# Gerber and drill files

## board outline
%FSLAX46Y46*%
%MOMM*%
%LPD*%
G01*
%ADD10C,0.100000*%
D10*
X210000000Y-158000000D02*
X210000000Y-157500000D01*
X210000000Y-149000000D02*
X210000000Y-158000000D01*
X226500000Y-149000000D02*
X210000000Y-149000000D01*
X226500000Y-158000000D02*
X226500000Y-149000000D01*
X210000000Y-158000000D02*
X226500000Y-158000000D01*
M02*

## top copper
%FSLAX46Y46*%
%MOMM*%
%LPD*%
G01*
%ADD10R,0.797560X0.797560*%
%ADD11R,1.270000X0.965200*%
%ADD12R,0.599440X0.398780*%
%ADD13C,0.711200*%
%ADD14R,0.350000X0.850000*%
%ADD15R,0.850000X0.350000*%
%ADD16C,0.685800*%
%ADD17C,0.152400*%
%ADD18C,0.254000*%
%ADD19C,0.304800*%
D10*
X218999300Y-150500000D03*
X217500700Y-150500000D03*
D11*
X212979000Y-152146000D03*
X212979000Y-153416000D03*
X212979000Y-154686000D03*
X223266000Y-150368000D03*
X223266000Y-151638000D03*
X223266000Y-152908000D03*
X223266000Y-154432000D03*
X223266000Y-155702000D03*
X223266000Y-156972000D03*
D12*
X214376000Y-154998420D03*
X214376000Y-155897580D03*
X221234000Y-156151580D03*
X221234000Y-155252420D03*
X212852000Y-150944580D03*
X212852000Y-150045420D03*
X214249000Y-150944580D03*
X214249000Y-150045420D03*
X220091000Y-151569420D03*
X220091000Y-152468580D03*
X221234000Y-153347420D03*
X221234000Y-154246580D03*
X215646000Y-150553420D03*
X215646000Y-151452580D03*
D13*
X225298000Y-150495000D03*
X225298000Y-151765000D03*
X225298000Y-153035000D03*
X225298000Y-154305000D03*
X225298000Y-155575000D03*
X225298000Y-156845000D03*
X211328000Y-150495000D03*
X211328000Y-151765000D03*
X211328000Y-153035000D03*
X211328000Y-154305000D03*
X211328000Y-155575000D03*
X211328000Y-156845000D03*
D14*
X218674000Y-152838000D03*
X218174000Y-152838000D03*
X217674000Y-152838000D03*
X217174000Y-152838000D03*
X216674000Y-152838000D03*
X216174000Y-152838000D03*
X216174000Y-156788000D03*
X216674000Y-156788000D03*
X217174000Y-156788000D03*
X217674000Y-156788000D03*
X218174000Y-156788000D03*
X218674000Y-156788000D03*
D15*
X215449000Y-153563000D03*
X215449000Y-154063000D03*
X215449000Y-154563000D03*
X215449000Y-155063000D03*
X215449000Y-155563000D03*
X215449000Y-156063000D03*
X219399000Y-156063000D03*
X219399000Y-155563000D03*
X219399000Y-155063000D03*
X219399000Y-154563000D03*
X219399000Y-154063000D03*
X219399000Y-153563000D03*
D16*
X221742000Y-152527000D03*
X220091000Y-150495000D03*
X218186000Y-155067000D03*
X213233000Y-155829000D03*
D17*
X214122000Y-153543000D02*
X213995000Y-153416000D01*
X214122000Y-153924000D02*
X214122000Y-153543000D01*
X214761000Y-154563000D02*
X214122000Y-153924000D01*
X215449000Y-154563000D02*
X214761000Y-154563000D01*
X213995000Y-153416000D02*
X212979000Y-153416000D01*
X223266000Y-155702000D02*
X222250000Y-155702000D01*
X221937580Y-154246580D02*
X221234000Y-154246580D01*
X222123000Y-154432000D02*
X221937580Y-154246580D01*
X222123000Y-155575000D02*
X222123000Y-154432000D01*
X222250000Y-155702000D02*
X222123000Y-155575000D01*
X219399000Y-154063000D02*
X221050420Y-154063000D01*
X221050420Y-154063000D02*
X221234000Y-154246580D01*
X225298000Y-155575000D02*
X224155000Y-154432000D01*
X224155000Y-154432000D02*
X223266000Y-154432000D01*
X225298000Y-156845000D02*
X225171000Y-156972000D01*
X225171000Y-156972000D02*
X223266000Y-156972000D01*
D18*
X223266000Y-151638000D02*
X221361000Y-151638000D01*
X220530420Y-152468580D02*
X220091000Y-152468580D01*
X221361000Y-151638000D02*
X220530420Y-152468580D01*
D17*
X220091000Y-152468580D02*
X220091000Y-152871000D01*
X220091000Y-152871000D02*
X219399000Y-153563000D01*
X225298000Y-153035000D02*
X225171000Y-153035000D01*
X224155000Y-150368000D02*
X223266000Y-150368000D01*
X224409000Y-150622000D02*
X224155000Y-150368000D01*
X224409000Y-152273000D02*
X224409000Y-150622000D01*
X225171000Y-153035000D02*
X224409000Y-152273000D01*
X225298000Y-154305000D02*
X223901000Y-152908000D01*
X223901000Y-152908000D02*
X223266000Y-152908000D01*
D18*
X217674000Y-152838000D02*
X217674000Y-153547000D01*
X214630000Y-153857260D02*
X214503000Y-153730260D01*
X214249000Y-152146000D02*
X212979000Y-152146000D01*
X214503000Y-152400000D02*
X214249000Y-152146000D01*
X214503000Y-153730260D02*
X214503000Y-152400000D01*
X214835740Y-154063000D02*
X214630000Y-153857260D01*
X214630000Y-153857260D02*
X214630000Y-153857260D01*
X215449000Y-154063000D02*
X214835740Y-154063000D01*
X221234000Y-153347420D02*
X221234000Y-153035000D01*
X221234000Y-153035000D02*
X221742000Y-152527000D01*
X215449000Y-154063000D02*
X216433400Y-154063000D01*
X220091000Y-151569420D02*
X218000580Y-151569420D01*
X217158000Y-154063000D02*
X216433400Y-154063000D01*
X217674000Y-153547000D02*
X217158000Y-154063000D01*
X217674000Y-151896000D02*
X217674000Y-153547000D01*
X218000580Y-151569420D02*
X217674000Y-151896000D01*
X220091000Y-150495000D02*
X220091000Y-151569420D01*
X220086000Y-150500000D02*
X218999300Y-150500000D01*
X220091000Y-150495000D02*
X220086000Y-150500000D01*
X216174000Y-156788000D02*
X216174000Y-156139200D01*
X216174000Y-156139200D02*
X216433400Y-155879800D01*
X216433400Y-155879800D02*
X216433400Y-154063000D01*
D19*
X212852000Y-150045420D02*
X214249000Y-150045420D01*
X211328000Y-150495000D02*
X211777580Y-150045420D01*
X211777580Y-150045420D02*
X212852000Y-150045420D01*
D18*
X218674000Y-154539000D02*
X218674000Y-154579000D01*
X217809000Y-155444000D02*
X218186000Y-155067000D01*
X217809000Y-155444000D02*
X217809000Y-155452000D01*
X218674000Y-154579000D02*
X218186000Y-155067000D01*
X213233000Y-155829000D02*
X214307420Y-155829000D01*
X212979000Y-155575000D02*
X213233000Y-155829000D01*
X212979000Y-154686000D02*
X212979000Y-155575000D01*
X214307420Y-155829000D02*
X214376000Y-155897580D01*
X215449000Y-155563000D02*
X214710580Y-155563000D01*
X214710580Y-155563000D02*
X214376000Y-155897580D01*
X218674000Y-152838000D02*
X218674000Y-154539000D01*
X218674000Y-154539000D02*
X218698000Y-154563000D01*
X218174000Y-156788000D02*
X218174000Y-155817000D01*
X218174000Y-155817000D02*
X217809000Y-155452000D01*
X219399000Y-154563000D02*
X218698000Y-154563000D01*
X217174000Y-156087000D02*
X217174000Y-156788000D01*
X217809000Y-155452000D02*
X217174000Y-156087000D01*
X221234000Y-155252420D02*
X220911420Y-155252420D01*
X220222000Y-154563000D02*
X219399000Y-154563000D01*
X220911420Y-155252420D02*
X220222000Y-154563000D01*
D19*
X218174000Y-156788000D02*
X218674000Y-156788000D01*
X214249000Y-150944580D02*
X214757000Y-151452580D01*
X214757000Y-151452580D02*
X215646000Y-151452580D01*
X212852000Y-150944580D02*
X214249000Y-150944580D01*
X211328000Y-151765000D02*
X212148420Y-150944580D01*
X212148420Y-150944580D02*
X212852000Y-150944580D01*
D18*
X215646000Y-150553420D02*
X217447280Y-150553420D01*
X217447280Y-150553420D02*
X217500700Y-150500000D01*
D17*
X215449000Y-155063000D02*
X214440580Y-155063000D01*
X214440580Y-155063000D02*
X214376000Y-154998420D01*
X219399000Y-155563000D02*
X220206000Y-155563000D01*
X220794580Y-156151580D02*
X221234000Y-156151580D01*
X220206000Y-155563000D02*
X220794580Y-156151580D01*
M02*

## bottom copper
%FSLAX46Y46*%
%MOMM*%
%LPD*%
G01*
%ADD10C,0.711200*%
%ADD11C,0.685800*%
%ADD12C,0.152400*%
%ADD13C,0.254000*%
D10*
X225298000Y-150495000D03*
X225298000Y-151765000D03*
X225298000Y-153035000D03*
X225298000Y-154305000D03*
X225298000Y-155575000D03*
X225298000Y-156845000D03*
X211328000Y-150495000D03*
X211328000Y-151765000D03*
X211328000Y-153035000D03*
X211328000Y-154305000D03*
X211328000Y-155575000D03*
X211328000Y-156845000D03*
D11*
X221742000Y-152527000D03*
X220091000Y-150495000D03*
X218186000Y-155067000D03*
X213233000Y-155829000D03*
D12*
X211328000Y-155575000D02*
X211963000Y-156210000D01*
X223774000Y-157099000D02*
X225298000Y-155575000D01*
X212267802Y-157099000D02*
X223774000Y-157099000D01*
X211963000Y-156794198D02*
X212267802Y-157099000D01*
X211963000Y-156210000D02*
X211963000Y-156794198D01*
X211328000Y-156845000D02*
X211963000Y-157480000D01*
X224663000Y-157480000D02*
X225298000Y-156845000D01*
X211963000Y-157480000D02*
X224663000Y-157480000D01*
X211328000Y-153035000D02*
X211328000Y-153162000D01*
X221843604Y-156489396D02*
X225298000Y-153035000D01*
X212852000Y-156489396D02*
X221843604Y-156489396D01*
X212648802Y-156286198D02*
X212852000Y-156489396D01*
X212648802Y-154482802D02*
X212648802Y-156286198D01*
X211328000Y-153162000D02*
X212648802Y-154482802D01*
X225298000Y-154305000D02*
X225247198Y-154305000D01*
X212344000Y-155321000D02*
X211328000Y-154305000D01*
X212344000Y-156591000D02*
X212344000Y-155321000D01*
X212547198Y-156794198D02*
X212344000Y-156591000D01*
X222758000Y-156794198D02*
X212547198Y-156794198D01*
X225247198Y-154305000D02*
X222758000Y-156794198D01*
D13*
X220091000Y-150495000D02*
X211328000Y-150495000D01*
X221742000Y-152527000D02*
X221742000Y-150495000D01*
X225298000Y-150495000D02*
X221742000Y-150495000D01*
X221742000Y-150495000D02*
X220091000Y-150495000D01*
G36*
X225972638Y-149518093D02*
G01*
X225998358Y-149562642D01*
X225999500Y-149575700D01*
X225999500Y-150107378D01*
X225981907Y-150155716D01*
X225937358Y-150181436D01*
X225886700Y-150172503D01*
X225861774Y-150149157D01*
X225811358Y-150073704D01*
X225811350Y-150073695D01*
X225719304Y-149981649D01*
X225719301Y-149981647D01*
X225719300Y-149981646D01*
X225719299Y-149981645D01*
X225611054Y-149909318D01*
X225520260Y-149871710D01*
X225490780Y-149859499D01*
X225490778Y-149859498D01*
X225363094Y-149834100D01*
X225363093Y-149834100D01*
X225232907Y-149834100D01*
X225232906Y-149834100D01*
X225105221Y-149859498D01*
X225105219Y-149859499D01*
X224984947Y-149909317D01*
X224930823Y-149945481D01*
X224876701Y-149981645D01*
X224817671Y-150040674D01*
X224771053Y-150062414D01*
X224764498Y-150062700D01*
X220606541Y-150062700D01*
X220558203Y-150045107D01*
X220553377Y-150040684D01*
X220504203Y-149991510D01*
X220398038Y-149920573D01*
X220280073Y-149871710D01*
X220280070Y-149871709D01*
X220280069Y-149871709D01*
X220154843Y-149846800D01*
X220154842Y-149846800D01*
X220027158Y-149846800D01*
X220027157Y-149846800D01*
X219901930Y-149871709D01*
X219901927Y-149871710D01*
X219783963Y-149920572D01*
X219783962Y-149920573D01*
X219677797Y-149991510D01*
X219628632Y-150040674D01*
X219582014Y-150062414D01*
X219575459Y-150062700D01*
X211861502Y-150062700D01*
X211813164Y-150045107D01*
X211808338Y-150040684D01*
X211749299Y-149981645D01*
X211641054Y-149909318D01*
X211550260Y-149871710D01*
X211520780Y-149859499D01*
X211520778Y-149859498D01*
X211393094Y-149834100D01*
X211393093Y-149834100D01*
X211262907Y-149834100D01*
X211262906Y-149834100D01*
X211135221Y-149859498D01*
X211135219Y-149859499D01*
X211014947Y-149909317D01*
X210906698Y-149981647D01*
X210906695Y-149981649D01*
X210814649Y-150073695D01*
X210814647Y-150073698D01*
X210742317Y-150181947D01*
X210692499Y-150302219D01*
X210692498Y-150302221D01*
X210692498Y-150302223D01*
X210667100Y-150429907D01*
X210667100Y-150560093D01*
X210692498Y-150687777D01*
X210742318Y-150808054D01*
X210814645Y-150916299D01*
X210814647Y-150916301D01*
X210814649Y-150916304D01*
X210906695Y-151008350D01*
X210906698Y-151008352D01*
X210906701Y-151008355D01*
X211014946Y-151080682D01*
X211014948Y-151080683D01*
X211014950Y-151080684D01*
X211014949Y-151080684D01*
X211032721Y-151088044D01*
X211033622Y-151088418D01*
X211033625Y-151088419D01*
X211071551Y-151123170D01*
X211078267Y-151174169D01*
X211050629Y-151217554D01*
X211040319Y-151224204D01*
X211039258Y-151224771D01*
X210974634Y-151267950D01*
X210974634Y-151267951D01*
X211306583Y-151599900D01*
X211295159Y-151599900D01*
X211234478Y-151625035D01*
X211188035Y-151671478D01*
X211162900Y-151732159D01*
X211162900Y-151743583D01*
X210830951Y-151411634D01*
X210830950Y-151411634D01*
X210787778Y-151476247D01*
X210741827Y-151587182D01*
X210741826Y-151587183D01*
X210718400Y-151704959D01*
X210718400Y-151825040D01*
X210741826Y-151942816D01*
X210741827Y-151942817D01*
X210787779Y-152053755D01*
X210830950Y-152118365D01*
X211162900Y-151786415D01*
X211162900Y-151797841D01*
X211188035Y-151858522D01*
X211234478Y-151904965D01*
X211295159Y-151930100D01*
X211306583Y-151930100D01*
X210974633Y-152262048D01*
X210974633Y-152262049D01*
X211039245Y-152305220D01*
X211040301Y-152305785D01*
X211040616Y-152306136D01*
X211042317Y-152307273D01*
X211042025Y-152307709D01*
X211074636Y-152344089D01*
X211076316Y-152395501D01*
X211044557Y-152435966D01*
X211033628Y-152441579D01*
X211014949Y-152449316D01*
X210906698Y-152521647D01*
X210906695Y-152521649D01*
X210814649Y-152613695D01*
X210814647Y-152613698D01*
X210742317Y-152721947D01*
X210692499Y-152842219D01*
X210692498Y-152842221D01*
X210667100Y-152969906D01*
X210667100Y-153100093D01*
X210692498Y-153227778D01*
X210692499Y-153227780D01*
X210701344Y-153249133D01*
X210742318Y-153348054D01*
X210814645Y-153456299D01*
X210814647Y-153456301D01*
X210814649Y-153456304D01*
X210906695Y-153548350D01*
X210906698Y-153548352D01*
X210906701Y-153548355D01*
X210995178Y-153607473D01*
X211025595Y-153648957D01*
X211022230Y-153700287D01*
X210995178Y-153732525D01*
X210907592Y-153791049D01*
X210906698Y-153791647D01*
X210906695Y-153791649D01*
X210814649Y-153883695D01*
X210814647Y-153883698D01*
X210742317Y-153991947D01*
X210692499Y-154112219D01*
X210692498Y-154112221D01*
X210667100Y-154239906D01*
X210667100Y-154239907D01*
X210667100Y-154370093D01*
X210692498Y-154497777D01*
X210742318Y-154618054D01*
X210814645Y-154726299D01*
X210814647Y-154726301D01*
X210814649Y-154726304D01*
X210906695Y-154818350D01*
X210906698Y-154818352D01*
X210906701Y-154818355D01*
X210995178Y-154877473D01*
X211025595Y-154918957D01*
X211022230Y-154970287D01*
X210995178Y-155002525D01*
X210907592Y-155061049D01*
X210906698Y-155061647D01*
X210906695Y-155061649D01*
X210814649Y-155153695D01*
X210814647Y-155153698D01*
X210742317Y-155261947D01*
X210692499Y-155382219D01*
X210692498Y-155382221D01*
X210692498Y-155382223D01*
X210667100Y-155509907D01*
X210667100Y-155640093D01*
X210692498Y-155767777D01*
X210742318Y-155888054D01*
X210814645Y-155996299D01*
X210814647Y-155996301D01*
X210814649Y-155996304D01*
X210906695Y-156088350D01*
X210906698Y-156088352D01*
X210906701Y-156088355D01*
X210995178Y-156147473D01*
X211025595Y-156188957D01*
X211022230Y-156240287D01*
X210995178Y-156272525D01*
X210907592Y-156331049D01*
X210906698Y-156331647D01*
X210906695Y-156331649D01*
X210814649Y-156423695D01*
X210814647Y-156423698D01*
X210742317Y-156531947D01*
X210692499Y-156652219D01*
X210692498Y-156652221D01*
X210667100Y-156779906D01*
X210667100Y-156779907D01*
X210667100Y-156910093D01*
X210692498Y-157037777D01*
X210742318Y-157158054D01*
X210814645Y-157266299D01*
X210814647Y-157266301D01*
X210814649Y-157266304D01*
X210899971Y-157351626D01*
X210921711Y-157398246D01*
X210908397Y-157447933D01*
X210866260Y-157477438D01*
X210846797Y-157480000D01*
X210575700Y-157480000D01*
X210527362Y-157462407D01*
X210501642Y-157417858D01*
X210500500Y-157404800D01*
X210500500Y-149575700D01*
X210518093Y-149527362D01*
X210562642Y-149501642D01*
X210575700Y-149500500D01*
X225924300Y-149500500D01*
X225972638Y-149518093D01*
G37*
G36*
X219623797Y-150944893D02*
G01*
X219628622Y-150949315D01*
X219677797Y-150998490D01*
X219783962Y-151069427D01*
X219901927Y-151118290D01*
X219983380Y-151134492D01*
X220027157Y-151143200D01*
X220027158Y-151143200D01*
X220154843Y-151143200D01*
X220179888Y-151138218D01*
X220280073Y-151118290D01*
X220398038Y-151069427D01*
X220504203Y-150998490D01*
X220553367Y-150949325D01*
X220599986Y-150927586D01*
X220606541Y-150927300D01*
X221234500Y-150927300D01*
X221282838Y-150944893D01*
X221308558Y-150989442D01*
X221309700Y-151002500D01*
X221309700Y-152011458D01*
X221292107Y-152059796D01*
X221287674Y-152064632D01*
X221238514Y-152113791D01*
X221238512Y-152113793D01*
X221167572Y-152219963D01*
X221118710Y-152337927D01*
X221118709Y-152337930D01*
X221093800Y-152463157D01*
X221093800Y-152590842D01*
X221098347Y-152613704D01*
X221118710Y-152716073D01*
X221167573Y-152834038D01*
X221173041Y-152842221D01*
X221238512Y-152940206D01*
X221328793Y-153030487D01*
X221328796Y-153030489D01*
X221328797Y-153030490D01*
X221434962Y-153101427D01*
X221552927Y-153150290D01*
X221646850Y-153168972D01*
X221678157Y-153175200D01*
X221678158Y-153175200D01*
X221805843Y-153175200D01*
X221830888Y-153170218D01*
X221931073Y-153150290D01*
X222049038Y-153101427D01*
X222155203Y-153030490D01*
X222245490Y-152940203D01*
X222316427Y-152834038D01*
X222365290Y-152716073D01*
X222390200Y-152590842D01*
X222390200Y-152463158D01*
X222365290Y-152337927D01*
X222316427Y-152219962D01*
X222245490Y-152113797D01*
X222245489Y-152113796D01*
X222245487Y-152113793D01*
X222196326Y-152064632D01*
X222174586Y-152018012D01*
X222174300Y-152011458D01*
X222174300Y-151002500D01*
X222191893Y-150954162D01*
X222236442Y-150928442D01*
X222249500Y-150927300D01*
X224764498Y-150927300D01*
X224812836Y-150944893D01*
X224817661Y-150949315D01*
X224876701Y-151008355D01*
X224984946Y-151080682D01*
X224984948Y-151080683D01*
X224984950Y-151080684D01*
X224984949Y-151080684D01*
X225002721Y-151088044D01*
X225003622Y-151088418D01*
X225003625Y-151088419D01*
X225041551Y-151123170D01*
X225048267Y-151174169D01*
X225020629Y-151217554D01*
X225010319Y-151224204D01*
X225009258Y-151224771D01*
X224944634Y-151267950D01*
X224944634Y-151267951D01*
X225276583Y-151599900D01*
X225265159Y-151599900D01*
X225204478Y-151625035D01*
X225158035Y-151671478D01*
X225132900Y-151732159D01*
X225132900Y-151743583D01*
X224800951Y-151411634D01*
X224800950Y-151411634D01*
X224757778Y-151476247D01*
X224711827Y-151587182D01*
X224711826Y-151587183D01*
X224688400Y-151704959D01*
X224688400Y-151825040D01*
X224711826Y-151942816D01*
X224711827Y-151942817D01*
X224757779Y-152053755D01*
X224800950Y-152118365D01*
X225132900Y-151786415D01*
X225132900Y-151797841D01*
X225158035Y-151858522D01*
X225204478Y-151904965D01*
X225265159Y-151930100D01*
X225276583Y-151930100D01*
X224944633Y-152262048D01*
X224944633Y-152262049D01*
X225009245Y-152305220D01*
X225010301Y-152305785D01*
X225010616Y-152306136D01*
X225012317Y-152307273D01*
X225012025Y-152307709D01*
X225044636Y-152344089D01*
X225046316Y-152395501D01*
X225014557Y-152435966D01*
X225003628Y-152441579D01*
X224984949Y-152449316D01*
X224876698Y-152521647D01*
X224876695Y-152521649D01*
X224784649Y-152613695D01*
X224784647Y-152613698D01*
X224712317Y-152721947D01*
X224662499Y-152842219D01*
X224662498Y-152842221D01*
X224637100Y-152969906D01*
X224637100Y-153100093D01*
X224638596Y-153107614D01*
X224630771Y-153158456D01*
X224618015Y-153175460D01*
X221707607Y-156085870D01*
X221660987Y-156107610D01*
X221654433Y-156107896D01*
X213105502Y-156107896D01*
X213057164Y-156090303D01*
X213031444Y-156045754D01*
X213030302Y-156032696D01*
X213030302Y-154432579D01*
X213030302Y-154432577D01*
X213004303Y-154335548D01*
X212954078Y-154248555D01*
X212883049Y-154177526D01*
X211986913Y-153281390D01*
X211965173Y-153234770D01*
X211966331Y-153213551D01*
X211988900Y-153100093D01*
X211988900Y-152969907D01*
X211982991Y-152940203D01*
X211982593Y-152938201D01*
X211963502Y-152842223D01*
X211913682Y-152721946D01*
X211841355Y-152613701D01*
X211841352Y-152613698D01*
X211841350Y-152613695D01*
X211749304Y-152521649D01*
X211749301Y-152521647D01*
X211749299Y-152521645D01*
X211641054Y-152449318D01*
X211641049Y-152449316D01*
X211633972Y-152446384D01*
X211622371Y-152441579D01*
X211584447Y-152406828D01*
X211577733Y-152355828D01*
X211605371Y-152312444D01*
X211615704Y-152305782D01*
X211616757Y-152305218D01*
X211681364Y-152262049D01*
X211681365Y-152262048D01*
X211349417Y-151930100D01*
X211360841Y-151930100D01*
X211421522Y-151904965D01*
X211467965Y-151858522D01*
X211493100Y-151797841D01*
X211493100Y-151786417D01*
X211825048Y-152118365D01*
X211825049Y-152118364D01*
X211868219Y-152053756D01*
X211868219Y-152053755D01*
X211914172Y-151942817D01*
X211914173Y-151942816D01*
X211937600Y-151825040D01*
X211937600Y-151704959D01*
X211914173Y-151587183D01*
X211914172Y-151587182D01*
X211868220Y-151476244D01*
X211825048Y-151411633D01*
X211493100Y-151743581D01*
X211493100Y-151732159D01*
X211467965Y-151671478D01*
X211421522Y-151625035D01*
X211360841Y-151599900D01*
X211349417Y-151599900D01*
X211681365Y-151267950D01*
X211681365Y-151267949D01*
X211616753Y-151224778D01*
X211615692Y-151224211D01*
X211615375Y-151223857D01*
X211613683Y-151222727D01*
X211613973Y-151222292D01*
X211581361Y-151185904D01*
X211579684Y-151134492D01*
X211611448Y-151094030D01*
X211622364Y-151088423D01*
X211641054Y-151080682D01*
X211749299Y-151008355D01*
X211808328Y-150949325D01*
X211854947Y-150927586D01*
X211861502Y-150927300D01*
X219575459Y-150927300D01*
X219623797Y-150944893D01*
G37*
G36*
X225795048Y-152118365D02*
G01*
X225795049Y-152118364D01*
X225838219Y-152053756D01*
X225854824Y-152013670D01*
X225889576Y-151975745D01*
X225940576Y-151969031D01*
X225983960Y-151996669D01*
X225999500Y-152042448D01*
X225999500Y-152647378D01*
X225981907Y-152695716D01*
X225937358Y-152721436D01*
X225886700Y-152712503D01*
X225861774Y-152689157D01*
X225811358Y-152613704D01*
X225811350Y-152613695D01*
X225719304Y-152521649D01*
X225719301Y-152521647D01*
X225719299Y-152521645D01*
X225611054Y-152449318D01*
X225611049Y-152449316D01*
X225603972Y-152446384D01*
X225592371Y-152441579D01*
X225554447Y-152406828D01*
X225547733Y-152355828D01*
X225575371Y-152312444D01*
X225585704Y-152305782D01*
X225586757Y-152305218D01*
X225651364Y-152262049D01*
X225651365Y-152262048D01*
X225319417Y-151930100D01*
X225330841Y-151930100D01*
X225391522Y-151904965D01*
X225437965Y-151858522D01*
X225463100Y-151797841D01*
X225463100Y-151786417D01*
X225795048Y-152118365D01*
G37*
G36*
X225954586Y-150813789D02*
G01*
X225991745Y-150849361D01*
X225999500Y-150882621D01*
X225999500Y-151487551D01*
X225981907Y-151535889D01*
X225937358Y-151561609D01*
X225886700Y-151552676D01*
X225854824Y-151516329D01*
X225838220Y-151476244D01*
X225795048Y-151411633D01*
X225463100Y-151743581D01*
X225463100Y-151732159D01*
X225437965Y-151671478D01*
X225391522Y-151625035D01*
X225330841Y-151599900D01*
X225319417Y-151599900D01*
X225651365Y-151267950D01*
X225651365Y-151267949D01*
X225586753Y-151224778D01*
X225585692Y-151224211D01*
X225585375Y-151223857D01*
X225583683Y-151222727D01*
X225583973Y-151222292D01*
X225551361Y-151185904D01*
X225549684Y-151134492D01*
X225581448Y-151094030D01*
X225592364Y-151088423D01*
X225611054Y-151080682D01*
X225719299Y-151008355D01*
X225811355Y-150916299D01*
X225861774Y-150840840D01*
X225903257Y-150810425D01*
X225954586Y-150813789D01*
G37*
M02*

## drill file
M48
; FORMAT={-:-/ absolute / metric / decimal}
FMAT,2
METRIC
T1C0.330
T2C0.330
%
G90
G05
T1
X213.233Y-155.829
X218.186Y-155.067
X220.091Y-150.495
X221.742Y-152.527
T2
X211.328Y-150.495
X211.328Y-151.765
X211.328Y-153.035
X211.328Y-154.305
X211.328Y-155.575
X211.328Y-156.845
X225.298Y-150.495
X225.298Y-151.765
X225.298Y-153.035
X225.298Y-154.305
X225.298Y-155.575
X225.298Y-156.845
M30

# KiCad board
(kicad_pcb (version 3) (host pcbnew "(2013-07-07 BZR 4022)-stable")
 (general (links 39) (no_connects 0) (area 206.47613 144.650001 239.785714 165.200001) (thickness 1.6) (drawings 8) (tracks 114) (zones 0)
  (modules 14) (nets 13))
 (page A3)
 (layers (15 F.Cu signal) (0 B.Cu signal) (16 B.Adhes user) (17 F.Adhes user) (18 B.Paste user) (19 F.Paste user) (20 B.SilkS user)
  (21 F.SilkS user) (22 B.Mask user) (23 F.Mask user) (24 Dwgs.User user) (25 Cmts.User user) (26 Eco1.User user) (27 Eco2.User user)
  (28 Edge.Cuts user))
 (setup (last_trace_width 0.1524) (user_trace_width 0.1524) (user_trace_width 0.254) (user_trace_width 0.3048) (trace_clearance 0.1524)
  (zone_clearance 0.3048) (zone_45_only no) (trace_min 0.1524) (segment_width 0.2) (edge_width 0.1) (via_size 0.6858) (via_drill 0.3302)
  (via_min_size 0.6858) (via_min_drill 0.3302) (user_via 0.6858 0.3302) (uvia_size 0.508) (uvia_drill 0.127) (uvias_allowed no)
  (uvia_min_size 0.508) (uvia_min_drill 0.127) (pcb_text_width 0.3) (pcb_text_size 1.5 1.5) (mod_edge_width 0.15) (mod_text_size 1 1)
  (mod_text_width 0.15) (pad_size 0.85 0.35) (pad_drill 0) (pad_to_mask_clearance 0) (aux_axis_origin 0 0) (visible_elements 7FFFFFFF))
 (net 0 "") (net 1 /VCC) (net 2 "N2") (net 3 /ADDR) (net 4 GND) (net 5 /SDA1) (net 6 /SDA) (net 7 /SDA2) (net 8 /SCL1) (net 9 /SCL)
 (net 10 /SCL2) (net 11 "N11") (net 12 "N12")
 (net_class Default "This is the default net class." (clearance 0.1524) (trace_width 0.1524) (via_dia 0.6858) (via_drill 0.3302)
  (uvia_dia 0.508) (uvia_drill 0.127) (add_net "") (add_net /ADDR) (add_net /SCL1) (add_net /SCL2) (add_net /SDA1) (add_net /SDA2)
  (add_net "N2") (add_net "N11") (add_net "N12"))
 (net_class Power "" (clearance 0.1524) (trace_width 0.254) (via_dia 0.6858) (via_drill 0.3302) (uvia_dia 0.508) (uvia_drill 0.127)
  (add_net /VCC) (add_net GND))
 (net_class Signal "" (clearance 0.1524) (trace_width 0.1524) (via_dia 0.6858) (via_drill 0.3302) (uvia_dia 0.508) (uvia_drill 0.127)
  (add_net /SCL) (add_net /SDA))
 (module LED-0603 (layer F.Cu) (at 218.25 150.5 180)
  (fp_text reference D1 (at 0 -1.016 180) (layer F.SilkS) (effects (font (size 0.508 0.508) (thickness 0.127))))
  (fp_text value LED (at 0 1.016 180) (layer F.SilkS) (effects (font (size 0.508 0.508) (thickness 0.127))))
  (pad 1 smd rect (at -0.7493 0 180) (size 0.79756 0.79756) (layers F.Cu F.Paste F.Mask) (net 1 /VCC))
  (pad 2 smd rect (at 0.7493 0 180) (size 0.79756 0.79756) (layers F.Cu F.Paste F.Mask) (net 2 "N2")))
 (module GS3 (layer F.Cu) (at 212.979 153.416)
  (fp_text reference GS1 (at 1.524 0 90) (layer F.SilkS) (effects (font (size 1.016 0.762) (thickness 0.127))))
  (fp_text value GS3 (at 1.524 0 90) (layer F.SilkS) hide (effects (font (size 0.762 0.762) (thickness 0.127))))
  (pad 1 smd rect (at 0 -1.27) (size 1.27 0.9652) (layers F.Cu F.Paste F.Mask) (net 1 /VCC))
  (pad 2 smd rect (at 0 0) (size 1.27 0.9652) (layers F.Cu F.Paste F.Mask) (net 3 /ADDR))
  (pad 3 smd rect (at 0 1.27) (size 1.27 0.9652) (layers F.Cu F.Paste F.Mask) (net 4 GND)))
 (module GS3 (layer F.Cu) (at 223.266 151.638)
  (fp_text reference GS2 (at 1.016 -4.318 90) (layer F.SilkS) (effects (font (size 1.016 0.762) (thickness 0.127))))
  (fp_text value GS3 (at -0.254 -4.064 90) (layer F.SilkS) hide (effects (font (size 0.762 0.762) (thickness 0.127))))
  (pad 1 smd rect (at 0 -1.27) (size 1.27 0.9652) (layers F.Cu F.Paste F.Mask) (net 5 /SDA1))
  (pad 2 smd rect (at 0 0) (size 1.27 0.9652) (layers F.Cu F.Paste F.Mask) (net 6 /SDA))
  (pad 3 smd rect (at 0 1.27) (size 1.27 0.9652) (layers F.Cu F.Paste F.Mask) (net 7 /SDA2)))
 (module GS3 (layer F.Cu) (at 223.266 155.702)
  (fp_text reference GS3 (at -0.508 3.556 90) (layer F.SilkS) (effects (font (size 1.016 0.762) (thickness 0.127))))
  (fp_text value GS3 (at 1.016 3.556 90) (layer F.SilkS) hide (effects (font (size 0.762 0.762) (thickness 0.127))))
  (pad 1 smd rect (at 0 -1.27) (size 1.27 0.9652) (layers F.Cu F.Paste F.Mask) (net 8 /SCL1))
  (pad 2 smd rect (at 0 0) (size 1.27 0.9652) (layers F.Cu F.Paste F.Mask) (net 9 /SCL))
  (pad 3 smd rect (at 0 1.27) (size 1.27 0.9652) (layers F.Cu F.Paste F.Mask) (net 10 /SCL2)))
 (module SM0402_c (layer F.Cu) (at 214.376 155.448 270)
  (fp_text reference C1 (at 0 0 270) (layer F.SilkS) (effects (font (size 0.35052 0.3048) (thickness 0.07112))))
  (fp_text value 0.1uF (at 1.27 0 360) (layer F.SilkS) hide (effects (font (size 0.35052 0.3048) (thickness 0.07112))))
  (pad 1 smd rect (at -0.44958 0 270) (size 0.39878 0.59944) (layers F.Cu F.Paste F.Mask) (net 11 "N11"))
  (pad 2 smd rect (at 0.44958 0 270) (size 0.39878 0.59944) (layers F.Cu F.Paste F.Mask) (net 4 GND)))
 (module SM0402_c (layer F.Cu) (at 221.234 155.702 90)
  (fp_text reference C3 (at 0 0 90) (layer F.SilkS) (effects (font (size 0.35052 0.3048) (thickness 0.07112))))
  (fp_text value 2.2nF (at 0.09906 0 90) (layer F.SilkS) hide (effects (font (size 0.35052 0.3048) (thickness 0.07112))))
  (pad 1 smd rect (at -0.44958 0 90) (size 0.39878 0.59944) (layers F.Cu F.Paste F.Mask) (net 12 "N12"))
  (pad 2 smd rect (at 0.44958 0 90) (size 0.39878 0.59944) (layers F.Cu F.Paste F.Mask) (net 4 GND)))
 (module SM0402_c (layer F.Cu) (at 212.852 150.495 90)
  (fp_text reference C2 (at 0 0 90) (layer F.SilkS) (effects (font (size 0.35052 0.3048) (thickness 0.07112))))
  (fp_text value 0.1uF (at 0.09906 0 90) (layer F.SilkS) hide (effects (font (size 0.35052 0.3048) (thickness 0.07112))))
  (pad 1 smd rect (at -0.44958 0 90) (size 0.39878 0.59944) (layers F.Cu F.Paste F.Mask) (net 4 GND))
  (pad 2 smd rect (at 0.44958 0 90) (size 0.39878 0.59944) (layers F.Cu F.Paste F.Mask) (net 1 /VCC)))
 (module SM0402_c (layer F.Cu) (at 214.249 150.495 90)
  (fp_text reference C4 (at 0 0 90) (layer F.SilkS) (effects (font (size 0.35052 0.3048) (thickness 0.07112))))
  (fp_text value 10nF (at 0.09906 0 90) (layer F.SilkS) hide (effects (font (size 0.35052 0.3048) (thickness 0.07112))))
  (pad 1 smd rect (at -0.44958 0 90) (size 0.39878 0.59944) (layers F.Cu F.Paste F.Mask) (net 4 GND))
  (pad 2 smd rect (at 0.44958 0 90) (size 0.39878 0.59944) (layers F.Cu F.Paste F.Mask) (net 1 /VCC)))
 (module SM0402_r (layer F.Cu) (at 220.091 152.019 270)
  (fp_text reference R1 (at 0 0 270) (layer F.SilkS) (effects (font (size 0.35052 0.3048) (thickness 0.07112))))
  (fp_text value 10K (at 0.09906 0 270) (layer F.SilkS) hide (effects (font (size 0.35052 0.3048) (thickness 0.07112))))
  (pad 1 smd rect (at -0.44958 0 270) (size 0.39878 0.59944) (layers F.Cu F.Paste F.Mask) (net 1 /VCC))
  (pad 2 smd rect (at 0.44958 0 270) (size 0.39878 0.59944) (layers F.Cu F.Paste F.Mask) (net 6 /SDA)))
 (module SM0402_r (layer F.Cu) (at 221.234 153.797 270)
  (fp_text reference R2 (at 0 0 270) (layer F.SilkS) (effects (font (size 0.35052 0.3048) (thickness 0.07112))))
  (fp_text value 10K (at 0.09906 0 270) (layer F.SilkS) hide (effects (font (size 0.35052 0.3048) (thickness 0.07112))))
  (pad 1 smd rect (at -0.44958 0 270) (size 0.39878 0.59944) (layers F.Cu F.Paste F.Mask) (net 1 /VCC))
  (pad 2 smd rect (at 0.44958 0 270) (size 0.39878 0.59944) (layers F.Cu F.Paste F.Mask) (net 9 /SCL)))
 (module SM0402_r (layer F.Cu) (at 215.646 151.003 270)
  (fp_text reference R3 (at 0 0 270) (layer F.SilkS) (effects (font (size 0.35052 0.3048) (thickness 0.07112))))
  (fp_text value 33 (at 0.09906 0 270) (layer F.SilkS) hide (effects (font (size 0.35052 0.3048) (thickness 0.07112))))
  (pad 1 smd rect (at -0.44958 0 270) (size 0.39878 0.59944) (layers F.Cu F.Paste F.Mask) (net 2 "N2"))
  (pad 2 smd rect (at 0.44958 0 270) (size 0.39878 0.59944) (layers F.Cu F.Paste F.Mask) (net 4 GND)))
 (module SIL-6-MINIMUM (layer F.Cu) (at 225.298 153.67 270)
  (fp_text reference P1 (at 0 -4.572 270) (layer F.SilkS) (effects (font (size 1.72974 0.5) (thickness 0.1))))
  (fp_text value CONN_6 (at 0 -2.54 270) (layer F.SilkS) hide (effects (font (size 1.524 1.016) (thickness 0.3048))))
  (pad 1 thru_hole circle (at -3.175 0 270) (size 0.7112 0.7112) (drill 0.3302) (layers *.Cu *.Mask F.SilkS) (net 1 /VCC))
  (pad 2 thru_hole circle (at -1.905 0 270) (size 0.7112 0.7112) (drill 0.3302) (layers *.Cu *.Mask F.SilkS) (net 4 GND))
  (pad 3 thru_hole circle (at -0.635 0 270) (size 0.7112 0.7112) (drill 0.3302) (layers *.Cu *.Mask F.SilkS) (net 5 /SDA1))
  (pad 4 thru_hole circle (at 0.635 0 270) (size 0.7112 0.7112) (drill 0.3302) (layers *.Cu *.Mask F.SilkS) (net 7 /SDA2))
  (pad 5 thru_hole circle (at 1.905 0 270) (size 0.7112 0.7112) (drill 0.3302) (layers *.Cu *.Mask F.SilkS) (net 8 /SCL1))
  (pad 6 thru_hole circle (at 3.175 0 270) (size 0.7112 0.7112) (drill 0.3302) (layers *.Cu *.Mask F.SilkS) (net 10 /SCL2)))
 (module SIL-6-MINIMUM (layer F.Cu) (at 211.328 153.67 270)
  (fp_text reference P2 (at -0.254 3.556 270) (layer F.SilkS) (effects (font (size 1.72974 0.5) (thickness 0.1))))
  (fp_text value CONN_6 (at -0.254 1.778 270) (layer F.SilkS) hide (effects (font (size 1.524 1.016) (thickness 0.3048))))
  (pad 1 thru_hole circle (at -3.175 0 270) (size 0.7112 0.7112) (drill 0.3302) (layers *.Cu *.Mask F.SilkS) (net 1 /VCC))
  (pad 2 thru_hole circle (at -1.905 0 270) (size 0.7112 0.7112) (drill 0.3302) (layers *.Cu *.Mask F.SilkS) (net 4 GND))
  (pad 3 thru_hole circle (at -0.635 0 270) (size 0.7112 0.7112) (drill 0.3302) (layers *.Cu *.Mask F.SilkS) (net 5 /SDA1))
  (pad 4 thru_hole circle (at 0.635 0 270) (size 0.7112 0.7112) (drill 0.3302) (layers *.Cu *.Mask F.SilkS) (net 7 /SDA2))
  (pad 5 thru_hole circle (at 1.905 0 270) (size 0.7112 0.7112) (drill 0.3302) (layers *.Cu *.Mask F.SilkS) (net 8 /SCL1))
  (pad 6 thru_hole circle (at 3.175 0 270) (size 0.7112 0.7112) (drill 0.3302) (layers *.Cu *.Mask F.SilkS) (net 10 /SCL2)))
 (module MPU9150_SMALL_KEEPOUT (layer F.Cu) (at 217.424 154.813 270)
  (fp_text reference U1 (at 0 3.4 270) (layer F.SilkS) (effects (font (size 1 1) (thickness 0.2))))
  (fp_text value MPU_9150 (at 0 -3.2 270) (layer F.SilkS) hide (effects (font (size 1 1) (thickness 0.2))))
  (pad 1 smd rect (at -1.975 -1.25 270) (size 0.85 0.35) (layers F.Cu F.Paste F.Mask) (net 4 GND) (clearance 0.0762))
  (pad 2 smd rect (at -1.975 -0.75 270) (size 0.85 0.35) (layers F.Cu F.Paste F.Mask) (clearance 0.0762))
  (pad 3 smd rect (at -1.975 -0.25 270) (size 0.85 0.35) (layers F.Cu F.Paste F.Mask) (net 1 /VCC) (clearance 0.0762))
  (pad 4 smd rect (at -1.975 0.25 270) (size 0.85 0.35) (layers F.Cu F.Paste F.Mask) (clearance 0.0762))
  (pad 5 smd rect (at -1.975 0.75 270) (size 0.85 0.35) (layers F.Cu F.Paste F.Mask) (clearance 0.0762))
  (pad 6 smd rect (at -1.975 1.25 270) (size 0.85 0.35) (layers F.Cu F.Paste F.Mask) (clearance 0.0762))
  (pad 13 smd rect (at 1.975 1.25 270) (size 0.85 0.35) (layers F.Cu F.Paste F.Mask) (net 1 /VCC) (clearance 0.0762))
  (pad 14 smd rect (at 1.975 0.75 270) (size 0.85 0.35) (layers F.Cu F.Paste F.Mask) (clearance 0.0762))
  (pad 15 smd rect (at 1.975 0.25 270) (size 0.85 0.35) (layers F.Cu F.Paste F.Mask) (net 4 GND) (clearance 0.0762))
  (pad 16 smd rect (at 1.975 -0.25 270) (size 0.85 0.35) (layers F.Cu F.Paste F.Mask) (clearance 0.0762))
  (pad 17 smd rect (at 1.975 -0.75 270) (size 0.85 0.35) (layers F.Cu F.Paste F.Mask) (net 4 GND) (clearance 0.0762))
  (pad 18 smd rect (at 1.975 -1.25 270) (size 0.85 0.35) (layers F.Cu F.Paste F.Mask) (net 4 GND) (clearance 0.0762))
  (pad 7 smd rect (at -1.25 1.975 270) (size 0.35 0.85) (layers F.Cu F.Paste F.Mask) (clearance 0.0762))
  (pad 8 smd rect (at -0.75 1.975 270) (size 0.35 0.85) (layers F.Cu F.Paste F.Mask) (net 1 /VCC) (clearance 0.0762))
  (pad 9 smd rect (at -0.25 1.975 270) (size 0.35 0.85) (layers F.Cu F.Paste F.Mask) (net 3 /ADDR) (clearance 0.0762))
  (pad 10 smd rect (at 0.25 1.975 270) (size 0.35 0.85) (layers F.Cu F.Paste F.Mask) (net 11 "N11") (clearance 0.0762))
  (pad 11 smd rect (at 0.75 1.975 270) (size 0.35 0.85) (layers F.Cu F.Paste F.Mask) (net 4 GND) (clearance 0.0762))
  (pad 12 smd rect (at 1.25 1.975 270) (size 0.35 0.85) (layers F.Cu F.Paste F.Mask) (clearance 0.0762))
  (pad 19 smd rect (at 1.25 -1.975 270) (size 0.35 0.85) (layers F.Cu F.Paste F.Mask) (clearance 0.0762))
  (pad 20 smd rect (at 0.75 -1.975 270) (size 0.35 0.85) (layers F.Cu F.Paste F.Mask) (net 12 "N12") (clearance 0.0762))
  (pad 21 smd rect (at 0.25 -1.975 270) (size 0.35 0.85) (layers F.Cu F.Paste F.Mask) (clearance 0.0762))
  (pad 22 smd rect (at -0.25 -1.975 270) (size 0.35 0.85) (layers F.Cu F.Paste F.Mask) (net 4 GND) (clearance 0.0762))
  (pad 23 smd rect (at -0.75 -1.975 270) (size 0.35 0.85) (layers F.Cu F.Paste F.Mask) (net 9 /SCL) (clearance 0.0762))
  (pad 24 smd rect (at -1.25 -1.975 270) (size 0.35 0.85) (layers F.Cu F.Paste F.Mask) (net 6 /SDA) (clearance 0.0762)))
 (gr_line (start 210 158) (end 210 157.5) (angle 90) (layer Edge.Cuts) (width 0.1))
 (gr_line (start 210 149) (end 210 158) (angle 90) (layer Edge.Cuts) (width 0.1))
 (gr_line (start 226.5 149) (end 210 149) (angle 90) (layer Edge.Cuts) (width 0.1))
 (gr_line (start 226.5 158) (end 226.5 149) (angle 90) (layer Edge.Cuts) (width 0.1))
 (gr_line (start 210 158) (end 226.5 158) (angle 90) (layer Edge.Cuts) (width 0.1))
 (segment (start 214.122 153.543) (end 213.995 153.416) (width 0.1524) (layer F.Cu) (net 3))
 (segment (start 214.122 153.924) (end 214.122 153.543) (width 0.1524) (layer F.Cu) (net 3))
 (segment (start 214.761 154.563) (end 214.122 153.924) (width 0.1524) (layer F.Cu) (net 3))
 (segment (start 215.449 154.563) (end 214.761 154.563) (width 0.1524) (layer F.Cu) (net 3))
 (segment (start 213.995 153.416) (end 212.979 153.416) (width 0.1524) (layer F.Cu) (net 3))
 (segment (start 223.266 155.702) (end 222.25 155.702) (width 0.1524) (layer F.Cu) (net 9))
 (segment (start 221.93758 154.24658) (end 221.234 154.24658) (width 0.1524) (layer F.Cu) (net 9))
 (segment (start 222.123 154.432) (end 221.93758 154.24658) (width 0.1524) (layer F.Cu) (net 9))
 (segment (start 222.123 155.575) (end 222.123 154.432) (width 0.1524) (layer F.Cu) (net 9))
 (segment (start 222.25 155.702) (end 222.123 155.575) (width 0.1524) (layer F.Cu) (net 9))
 (segment (start 219.399 154.063) (end 221.05042 154.063) (width 0.1524) (layer F.Cu) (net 9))
 (segment (start 221.05042 154.063) (end 221.234 154.24658) (width 0.1524) (layer F.Cu) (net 9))
 (segment (start 211.328 155.575) (end 211.963 156.21) (width 0.1524) (layer B.Cu) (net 8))
 (segment (start 223.774 157.099) (end 225.298 155.575) (width 0.1524) (layer B.Cu) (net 8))
 (segment (start 212.267802 157.099) (end 223.774 157.099) (width 0.1524) (layer B.Cu) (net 8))
 (segment (start 211.963 156.794198) (end 212.267802 157.099) (width 0.1524) (layer B.Cu) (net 8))
 (segment (start 211.963 156.21) (end 211.963 156.794198) (width 0.1524) (layer B.Cu) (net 8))
 (segment (start 225.298 155.575) (end 224.155 154.432) (width 0.1524) (layer F.Cu) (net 8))
 (segment (start 224.155 154.432) (end 223.266 154.432) (width 0.1524) (layer F.Cu) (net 8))
 (segment (start 211.328 156.845) (end 211.963 157.48) (width 0.1524) (layer B.Cu) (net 10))
 (segment (start 224.663 157.48) (end 225.298 156.845) (width 0.1524) (layer B.Cu) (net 10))
 (segment (start 211.963 157.48) (end 224.663 157.48) (width 0.1524) (layer B.Cu) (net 10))
 (segment (start 225.298 156.845) (end 225.171 156.972) (width 0.1524) (layer F.Cu) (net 10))
 (segment (start 225.171 156.972) (end 223.266 156.972) (width 0.1524) (layer F.Cu) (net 10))
 (segment (start 223.266 151.638) (end 221.361 151.638) (width 0.254) (layer F.Cu) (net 6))
 (segment (start 220.53042 152.46858) (end 220.091 152.46858) (width 0.254) (layer F.Cu) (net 6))
 (segment (start 221.361 151.638) (end 220.53042 152.46858) (width 0.254) (layer F.Cu) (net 6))
 (segment (start 220.091 152.46858) (end 220.091 152.871) (width 0.1524) (layer F.Cu) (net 6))
 (segment (start 220.091 152.871) (end 219.399 153.563) (width 0.1524) (layer F.Cu) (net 6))
 (segment (start 211.328 153.035) (end 211.328 153.162) (width 0.1524) (layer B.Cu) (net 5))
 (segment (start 221.843604 156.489396) (end 225.298 153.035) (width 0.1524) (layer B.Cu) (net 5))
 (segment (start 212.852 156.489396) (end 221.843604 156.489396) (width 0.1524) (layer B.Cu) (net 5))
 (segment (start 212.648802 156.286198) (end 212.852 156.489396) (width 0.1524) (layer B.Cu) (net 5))
 (segment (start 212.648802 154.482802) (end 212.648802 156.286198) (width 0.1524) (layer B.Cu) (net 5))
 (segment (start 211.328 153.162) (end 212.648802 154.482802) (width 0.1524) (layer B.Cu) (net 5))
 (segment (start 225.298 153.035) (end 225.171 153.035) (width 0.1524) (layer F.Cu) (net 5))
 (segment (start 224.155 150.368) (end 223.266 150.368) (width 0.1524) (layer F.Cu) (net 5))
 (segment (start 224.409 150.622) (end 224.155 150.368) (width 0.1524) (layer F.Cu) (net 5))
 (segment (start 224.409 152.273) (end 224.409 150.622) (width 0.1524) (layer F.Cu) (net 5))
 (segment (start 225.171 153.035) (end 224.409 152.273) (width 0.1524) (layer F.Cu) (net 5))
 (segment (start 225.298 154.305) (end 225.247198 154.305) (width 0.1524) (layer B.Cu) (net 7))
 (segment (start 212.344 155.321) (end 211.328 154.305) (width 0.1524) (layer B.Cu) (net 7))
 (segment (start 212.344 156.591) (end 212.344 155.321) (width 0.1524) (layer B.Cu) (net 7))
 (segment (start 212.547198 156.794198) (end 212.344 156.591) (width 0.1524) (layer B.Cu) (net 7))
 (segment (start 222.758 156.794198) (end 212.547198 156.794198) (width 0.1524) (layer B.Cu) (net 7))
 (segment (start 225.247198 154.305) (end 222.758 156.794198) (width 0.1524) (layer B.Cu) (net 7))
 (segment (start 225.298 154.305) (end 223.901 152.908) (width 0.1524) (layer F.Cu) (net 7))
 (segment (start 223.901 152.908) (end 223.266 152.908) (width 0.1524) (layer F.Cu) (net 7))
 (segment (start 217.674 152.838) (end 217.674 153.547) (width 0.254) (layer F.Cu) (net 1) (status 400000))
 (segment (start 214.63 153.85726) (end 214.503 153.73026) (width 0.254) (layer F.Cu) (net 1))
 (segment (start 214.249 152.146) (end 212.979 152.146) (width 0.254) (layer F.Cu) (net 1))
 (segment (start 214.503 152.4) (end 214.249 152.146) (width 0.254) (layer F.Cu) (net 1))
 (segment (start 214.503 153.73026) (end 214.503 152.4) (width 0.254) (layer F.Cu) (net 1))
 (segment (start 214.83574 154.063) (end 214.63 153.85726) (width 0.254) (layer F.Cu) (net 1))
 (segment (start 214.63 153.85726) (end 214.63 153.85726) (width 0.254) (layer F.Cu) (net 1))
 (segment (start 215.449 154.063) (end 214.83574 154.063) (width 0.254) (layer F.Cu) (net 1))
 (segment (start 220.091 150.495) (end 211.328 150.495) (width 0.254) (layer B.Cu) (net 1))
 (segment (start 221.234 153.34742) (end 221.234 153.035) (width 0.254) (layer F.Cu) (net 1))
 (segment (start 221.742 152.527) (end 221.742 150.495) (width 0.254) (layer B.Cu) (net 1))
 (via (at 221.742 152.527) (size 0.6858) (layers F.Cu B.Cu) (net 1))
 (segment (start 221.234 153.035) (end 221.742 152.527) (width 0.254) (layer F.Cu) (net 1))
 (segment (start 215.449 154.063) (end 216.4334 154.063) (width 0.254) (layer F.Cu) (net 1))
 (segment (start 220.091 151.56942) (end 218.00058 151.56942) (width 0.254) (layer F.Cu) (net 1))
 (segment (start 217.158 154.063) (end 216.4334 154.063) (width 0.254) (layer F.Cu) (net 1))
 (segment (start 217.674 153.547) (end 217.158 154.063) (width 0.254) (layer F.Cu) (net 1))
 (segment (start 217.674 151.896) (end 217.674 153.547) (width 0.254) (layer F.Cu) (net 1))
 (segment (start 218.00058 151.56942) (end 217.674 151.896) (width 0.254) (layer F.Cu) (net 1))
 (segment (start 220.091 150.495) (end 220.091 151.56942) (width 0.254) (layer F.Cu) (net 1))
 (segment (start 225.298 150.495) (end 221.742 150.495) (width 0.254) (layer B.Cu) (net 1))
 (segment (start 221.742 150.495) (end 220.091 150.495) (width 0.254) (layer B.Cu) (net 1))
 (segment (start 220.086 150.5) (end 218.9993 150.5) (width 0.254) (layer F.Cu) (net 1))
 (segment (start 220.091 150.495) (end 220.086 150.5) (width 0.254) (layer F.Cu) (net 1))
 (via (at 220.091 150.495) (size 0.6858) (layers F.Cu B.Cu) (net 1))
 (segment (start 216.174 156.788) (end 216.174 156.1392) (width 0.254) (layer F.Cu) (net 1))
 (segment (start 216.174 156.1392) (end 216.4334 155.8798) (width 0.254) (layer F.Cu) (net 1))
 (segment (start 216.4334 155.8798) (end 216.4334 154.063) (width 0.254) (layer F.Cu) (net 1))
 (segment (start 212.852 150.04542) (end 214.249 150.04542) (width 0.3048) (layer F.Cu) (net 1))
 (segment (start 211.328 150.495) (end 211.77758 150.04542) (width 0.3048) (layer F.Cu) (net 1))
 (segment (start 211.77758 150.04542) (end 212.852 150.04542) (width 0.3048) (layer F.Cu) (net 1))
 (segment (start 218.674 154.539) (end 218.674 154.579) (width 0.254) (layer F.Cu) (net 4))
 (segment (start 217.809 155.444) (end 218.186 155.067) (width 0.254) (layer F.Cu) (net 4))
 (via (at 218.186 155.067) (size 0.6858) (layers F.Cu B.Cu) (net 4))
 (segment (start 217.809 155.444) (end 217.809 155.452) (width 0.254) (layer F.Cu) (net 4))
 (segment (start 218.674 154.579) (end 218.186 155.067) (width 0.254) (layer F.Cu) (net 4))
 (segment (start 213.233 155.829) (end 214.30742 155.829) (width 0.254) (layer F.Cu) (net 4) (status 800000))
 (segment (start 212.979 155.575) (end 213.233 155.829) (width 0.254) (layer F.Cu) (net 4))
 (via (at 213.233 155.829) (size 0.6858) (layers F.Cu B.Cu) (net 4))
 (segment (start 212.979 154.686) (end 212.979 155.575) (width 0.254) (layer F.Cu) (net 4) (status 400000))
 (segment (start 214.30742 155.829) (end 214.376 155.89758) (width 0.254) (layer F.Cu) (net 4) (status C00000))
 (segment (start 215.449 155.563) (end 214.71058 155.563) (width 0.254) (layer F.Cu) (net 4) (status 400000))
 (segment (start 214.71058 155.563) (end 214.376 155.89758) (width 0.254) (layer F.Cu) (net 4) (status 800000))
 (segment (start 218.674 152.838) (end 218.674 154.539) (width 0.254) (layer F.Cu) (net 4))
 (segment (start 218.674 154.539) (end 218.698 154.563) (width 0.254) (layer F.Cu) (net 4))
 (segment (start 218.174 156.788) (end 218.174 155.817) (width 0.254) (layer F.Cu) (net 4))
 (segment (start 218.174 155.817) (end 217.809 155.452) (width 0.254) (layer F.Cu) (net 4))
 (segment (start 219.399 154.563) (end 218.698 154.563) (width 0.254) (layer F.Cu) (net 4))
 (segment (start 217.174 156.087) (end 217.174 156.788) (width 0.254) (layer F.Cu) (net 4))
 (segment (start 217.809 155.452) (end 217.174 156.087) (width 0.254) (layer F.Cu) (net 4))
 (segment (start 221.234 155.25242) (end 220.91142 155.25242) (width 0.254) (layer F.Cu) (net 4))
 (segment (start 220.222 154.563) (end 219.399 154.563) (width 0.254) (layer F.Cu) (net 4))
 (segment (start 220.91142 155.25242) (end 220.222 154.563) (width 0.254) (layer F.Cu) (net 4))
 (segment (start 218.174 156.788) (end 218.674 156.788) (width 0.3048) (layer F.Cu) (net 4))
 (segment (start 214.249 150.94458) (end 214.757 151.45258) (width 0.3048) (layer F.Cu) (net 4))
 (segment (start 214.757 151.45258) (end 215.646 151.45258) (width 0.3048) (layer F.Cu) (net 4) (status 20))
 (segment (start 212.852 150.94458) (end 214.249 150.94458) (width 0.3048) (layer F.Cu) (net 4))
 (segment (start 211.328 151.765) (end 212.14842 150.94458) (width 0.3048) (layer F.Cu) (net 4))
 (segment (start 212.14842 150.94458) (end 212.852 150.94458) (width 0.3048) (layer F.Cu) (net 4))
 (segment (start 215.646 150.55342) (end 217.44728 150.55342) (width 0.254) (layer F.Cu) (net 2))
 (segment (start 217.44728 150.55342) (end 217.5007 150.5) (width 0.254) (layer F.Cu) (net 2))
 (segment (start 215.449 155.063) (end 214.44058 155.063) (width 0.1524) (layer F.Cu) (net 11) (status 20))
 (segment (start 214.44058 155.063) (end 214.376 154.99842) (width 0.1524) (layer F.Cu) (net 11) (status 30))
 (segment (start 219.399 155.563) (end 220.206 155.563) (width 0.1524) (layer F.Cu) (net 12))
 (segment (start 220.79458 156.15158) (end 221.234 156.15158) (width 0.1524) (layer F.Cu) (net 12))
 (segment (start 220.206 155.563) (end 220.79458 156.15158) (width 0.1524) (layer F.Cu) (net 12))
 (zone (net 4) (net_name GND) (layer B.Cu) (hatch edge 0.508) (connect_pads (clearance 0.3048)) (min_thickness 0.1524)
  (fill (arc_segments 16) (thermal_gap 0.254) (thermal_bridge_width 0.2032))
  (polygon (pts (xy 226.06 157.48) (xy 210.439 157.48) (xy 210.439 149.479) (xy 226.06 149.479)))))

